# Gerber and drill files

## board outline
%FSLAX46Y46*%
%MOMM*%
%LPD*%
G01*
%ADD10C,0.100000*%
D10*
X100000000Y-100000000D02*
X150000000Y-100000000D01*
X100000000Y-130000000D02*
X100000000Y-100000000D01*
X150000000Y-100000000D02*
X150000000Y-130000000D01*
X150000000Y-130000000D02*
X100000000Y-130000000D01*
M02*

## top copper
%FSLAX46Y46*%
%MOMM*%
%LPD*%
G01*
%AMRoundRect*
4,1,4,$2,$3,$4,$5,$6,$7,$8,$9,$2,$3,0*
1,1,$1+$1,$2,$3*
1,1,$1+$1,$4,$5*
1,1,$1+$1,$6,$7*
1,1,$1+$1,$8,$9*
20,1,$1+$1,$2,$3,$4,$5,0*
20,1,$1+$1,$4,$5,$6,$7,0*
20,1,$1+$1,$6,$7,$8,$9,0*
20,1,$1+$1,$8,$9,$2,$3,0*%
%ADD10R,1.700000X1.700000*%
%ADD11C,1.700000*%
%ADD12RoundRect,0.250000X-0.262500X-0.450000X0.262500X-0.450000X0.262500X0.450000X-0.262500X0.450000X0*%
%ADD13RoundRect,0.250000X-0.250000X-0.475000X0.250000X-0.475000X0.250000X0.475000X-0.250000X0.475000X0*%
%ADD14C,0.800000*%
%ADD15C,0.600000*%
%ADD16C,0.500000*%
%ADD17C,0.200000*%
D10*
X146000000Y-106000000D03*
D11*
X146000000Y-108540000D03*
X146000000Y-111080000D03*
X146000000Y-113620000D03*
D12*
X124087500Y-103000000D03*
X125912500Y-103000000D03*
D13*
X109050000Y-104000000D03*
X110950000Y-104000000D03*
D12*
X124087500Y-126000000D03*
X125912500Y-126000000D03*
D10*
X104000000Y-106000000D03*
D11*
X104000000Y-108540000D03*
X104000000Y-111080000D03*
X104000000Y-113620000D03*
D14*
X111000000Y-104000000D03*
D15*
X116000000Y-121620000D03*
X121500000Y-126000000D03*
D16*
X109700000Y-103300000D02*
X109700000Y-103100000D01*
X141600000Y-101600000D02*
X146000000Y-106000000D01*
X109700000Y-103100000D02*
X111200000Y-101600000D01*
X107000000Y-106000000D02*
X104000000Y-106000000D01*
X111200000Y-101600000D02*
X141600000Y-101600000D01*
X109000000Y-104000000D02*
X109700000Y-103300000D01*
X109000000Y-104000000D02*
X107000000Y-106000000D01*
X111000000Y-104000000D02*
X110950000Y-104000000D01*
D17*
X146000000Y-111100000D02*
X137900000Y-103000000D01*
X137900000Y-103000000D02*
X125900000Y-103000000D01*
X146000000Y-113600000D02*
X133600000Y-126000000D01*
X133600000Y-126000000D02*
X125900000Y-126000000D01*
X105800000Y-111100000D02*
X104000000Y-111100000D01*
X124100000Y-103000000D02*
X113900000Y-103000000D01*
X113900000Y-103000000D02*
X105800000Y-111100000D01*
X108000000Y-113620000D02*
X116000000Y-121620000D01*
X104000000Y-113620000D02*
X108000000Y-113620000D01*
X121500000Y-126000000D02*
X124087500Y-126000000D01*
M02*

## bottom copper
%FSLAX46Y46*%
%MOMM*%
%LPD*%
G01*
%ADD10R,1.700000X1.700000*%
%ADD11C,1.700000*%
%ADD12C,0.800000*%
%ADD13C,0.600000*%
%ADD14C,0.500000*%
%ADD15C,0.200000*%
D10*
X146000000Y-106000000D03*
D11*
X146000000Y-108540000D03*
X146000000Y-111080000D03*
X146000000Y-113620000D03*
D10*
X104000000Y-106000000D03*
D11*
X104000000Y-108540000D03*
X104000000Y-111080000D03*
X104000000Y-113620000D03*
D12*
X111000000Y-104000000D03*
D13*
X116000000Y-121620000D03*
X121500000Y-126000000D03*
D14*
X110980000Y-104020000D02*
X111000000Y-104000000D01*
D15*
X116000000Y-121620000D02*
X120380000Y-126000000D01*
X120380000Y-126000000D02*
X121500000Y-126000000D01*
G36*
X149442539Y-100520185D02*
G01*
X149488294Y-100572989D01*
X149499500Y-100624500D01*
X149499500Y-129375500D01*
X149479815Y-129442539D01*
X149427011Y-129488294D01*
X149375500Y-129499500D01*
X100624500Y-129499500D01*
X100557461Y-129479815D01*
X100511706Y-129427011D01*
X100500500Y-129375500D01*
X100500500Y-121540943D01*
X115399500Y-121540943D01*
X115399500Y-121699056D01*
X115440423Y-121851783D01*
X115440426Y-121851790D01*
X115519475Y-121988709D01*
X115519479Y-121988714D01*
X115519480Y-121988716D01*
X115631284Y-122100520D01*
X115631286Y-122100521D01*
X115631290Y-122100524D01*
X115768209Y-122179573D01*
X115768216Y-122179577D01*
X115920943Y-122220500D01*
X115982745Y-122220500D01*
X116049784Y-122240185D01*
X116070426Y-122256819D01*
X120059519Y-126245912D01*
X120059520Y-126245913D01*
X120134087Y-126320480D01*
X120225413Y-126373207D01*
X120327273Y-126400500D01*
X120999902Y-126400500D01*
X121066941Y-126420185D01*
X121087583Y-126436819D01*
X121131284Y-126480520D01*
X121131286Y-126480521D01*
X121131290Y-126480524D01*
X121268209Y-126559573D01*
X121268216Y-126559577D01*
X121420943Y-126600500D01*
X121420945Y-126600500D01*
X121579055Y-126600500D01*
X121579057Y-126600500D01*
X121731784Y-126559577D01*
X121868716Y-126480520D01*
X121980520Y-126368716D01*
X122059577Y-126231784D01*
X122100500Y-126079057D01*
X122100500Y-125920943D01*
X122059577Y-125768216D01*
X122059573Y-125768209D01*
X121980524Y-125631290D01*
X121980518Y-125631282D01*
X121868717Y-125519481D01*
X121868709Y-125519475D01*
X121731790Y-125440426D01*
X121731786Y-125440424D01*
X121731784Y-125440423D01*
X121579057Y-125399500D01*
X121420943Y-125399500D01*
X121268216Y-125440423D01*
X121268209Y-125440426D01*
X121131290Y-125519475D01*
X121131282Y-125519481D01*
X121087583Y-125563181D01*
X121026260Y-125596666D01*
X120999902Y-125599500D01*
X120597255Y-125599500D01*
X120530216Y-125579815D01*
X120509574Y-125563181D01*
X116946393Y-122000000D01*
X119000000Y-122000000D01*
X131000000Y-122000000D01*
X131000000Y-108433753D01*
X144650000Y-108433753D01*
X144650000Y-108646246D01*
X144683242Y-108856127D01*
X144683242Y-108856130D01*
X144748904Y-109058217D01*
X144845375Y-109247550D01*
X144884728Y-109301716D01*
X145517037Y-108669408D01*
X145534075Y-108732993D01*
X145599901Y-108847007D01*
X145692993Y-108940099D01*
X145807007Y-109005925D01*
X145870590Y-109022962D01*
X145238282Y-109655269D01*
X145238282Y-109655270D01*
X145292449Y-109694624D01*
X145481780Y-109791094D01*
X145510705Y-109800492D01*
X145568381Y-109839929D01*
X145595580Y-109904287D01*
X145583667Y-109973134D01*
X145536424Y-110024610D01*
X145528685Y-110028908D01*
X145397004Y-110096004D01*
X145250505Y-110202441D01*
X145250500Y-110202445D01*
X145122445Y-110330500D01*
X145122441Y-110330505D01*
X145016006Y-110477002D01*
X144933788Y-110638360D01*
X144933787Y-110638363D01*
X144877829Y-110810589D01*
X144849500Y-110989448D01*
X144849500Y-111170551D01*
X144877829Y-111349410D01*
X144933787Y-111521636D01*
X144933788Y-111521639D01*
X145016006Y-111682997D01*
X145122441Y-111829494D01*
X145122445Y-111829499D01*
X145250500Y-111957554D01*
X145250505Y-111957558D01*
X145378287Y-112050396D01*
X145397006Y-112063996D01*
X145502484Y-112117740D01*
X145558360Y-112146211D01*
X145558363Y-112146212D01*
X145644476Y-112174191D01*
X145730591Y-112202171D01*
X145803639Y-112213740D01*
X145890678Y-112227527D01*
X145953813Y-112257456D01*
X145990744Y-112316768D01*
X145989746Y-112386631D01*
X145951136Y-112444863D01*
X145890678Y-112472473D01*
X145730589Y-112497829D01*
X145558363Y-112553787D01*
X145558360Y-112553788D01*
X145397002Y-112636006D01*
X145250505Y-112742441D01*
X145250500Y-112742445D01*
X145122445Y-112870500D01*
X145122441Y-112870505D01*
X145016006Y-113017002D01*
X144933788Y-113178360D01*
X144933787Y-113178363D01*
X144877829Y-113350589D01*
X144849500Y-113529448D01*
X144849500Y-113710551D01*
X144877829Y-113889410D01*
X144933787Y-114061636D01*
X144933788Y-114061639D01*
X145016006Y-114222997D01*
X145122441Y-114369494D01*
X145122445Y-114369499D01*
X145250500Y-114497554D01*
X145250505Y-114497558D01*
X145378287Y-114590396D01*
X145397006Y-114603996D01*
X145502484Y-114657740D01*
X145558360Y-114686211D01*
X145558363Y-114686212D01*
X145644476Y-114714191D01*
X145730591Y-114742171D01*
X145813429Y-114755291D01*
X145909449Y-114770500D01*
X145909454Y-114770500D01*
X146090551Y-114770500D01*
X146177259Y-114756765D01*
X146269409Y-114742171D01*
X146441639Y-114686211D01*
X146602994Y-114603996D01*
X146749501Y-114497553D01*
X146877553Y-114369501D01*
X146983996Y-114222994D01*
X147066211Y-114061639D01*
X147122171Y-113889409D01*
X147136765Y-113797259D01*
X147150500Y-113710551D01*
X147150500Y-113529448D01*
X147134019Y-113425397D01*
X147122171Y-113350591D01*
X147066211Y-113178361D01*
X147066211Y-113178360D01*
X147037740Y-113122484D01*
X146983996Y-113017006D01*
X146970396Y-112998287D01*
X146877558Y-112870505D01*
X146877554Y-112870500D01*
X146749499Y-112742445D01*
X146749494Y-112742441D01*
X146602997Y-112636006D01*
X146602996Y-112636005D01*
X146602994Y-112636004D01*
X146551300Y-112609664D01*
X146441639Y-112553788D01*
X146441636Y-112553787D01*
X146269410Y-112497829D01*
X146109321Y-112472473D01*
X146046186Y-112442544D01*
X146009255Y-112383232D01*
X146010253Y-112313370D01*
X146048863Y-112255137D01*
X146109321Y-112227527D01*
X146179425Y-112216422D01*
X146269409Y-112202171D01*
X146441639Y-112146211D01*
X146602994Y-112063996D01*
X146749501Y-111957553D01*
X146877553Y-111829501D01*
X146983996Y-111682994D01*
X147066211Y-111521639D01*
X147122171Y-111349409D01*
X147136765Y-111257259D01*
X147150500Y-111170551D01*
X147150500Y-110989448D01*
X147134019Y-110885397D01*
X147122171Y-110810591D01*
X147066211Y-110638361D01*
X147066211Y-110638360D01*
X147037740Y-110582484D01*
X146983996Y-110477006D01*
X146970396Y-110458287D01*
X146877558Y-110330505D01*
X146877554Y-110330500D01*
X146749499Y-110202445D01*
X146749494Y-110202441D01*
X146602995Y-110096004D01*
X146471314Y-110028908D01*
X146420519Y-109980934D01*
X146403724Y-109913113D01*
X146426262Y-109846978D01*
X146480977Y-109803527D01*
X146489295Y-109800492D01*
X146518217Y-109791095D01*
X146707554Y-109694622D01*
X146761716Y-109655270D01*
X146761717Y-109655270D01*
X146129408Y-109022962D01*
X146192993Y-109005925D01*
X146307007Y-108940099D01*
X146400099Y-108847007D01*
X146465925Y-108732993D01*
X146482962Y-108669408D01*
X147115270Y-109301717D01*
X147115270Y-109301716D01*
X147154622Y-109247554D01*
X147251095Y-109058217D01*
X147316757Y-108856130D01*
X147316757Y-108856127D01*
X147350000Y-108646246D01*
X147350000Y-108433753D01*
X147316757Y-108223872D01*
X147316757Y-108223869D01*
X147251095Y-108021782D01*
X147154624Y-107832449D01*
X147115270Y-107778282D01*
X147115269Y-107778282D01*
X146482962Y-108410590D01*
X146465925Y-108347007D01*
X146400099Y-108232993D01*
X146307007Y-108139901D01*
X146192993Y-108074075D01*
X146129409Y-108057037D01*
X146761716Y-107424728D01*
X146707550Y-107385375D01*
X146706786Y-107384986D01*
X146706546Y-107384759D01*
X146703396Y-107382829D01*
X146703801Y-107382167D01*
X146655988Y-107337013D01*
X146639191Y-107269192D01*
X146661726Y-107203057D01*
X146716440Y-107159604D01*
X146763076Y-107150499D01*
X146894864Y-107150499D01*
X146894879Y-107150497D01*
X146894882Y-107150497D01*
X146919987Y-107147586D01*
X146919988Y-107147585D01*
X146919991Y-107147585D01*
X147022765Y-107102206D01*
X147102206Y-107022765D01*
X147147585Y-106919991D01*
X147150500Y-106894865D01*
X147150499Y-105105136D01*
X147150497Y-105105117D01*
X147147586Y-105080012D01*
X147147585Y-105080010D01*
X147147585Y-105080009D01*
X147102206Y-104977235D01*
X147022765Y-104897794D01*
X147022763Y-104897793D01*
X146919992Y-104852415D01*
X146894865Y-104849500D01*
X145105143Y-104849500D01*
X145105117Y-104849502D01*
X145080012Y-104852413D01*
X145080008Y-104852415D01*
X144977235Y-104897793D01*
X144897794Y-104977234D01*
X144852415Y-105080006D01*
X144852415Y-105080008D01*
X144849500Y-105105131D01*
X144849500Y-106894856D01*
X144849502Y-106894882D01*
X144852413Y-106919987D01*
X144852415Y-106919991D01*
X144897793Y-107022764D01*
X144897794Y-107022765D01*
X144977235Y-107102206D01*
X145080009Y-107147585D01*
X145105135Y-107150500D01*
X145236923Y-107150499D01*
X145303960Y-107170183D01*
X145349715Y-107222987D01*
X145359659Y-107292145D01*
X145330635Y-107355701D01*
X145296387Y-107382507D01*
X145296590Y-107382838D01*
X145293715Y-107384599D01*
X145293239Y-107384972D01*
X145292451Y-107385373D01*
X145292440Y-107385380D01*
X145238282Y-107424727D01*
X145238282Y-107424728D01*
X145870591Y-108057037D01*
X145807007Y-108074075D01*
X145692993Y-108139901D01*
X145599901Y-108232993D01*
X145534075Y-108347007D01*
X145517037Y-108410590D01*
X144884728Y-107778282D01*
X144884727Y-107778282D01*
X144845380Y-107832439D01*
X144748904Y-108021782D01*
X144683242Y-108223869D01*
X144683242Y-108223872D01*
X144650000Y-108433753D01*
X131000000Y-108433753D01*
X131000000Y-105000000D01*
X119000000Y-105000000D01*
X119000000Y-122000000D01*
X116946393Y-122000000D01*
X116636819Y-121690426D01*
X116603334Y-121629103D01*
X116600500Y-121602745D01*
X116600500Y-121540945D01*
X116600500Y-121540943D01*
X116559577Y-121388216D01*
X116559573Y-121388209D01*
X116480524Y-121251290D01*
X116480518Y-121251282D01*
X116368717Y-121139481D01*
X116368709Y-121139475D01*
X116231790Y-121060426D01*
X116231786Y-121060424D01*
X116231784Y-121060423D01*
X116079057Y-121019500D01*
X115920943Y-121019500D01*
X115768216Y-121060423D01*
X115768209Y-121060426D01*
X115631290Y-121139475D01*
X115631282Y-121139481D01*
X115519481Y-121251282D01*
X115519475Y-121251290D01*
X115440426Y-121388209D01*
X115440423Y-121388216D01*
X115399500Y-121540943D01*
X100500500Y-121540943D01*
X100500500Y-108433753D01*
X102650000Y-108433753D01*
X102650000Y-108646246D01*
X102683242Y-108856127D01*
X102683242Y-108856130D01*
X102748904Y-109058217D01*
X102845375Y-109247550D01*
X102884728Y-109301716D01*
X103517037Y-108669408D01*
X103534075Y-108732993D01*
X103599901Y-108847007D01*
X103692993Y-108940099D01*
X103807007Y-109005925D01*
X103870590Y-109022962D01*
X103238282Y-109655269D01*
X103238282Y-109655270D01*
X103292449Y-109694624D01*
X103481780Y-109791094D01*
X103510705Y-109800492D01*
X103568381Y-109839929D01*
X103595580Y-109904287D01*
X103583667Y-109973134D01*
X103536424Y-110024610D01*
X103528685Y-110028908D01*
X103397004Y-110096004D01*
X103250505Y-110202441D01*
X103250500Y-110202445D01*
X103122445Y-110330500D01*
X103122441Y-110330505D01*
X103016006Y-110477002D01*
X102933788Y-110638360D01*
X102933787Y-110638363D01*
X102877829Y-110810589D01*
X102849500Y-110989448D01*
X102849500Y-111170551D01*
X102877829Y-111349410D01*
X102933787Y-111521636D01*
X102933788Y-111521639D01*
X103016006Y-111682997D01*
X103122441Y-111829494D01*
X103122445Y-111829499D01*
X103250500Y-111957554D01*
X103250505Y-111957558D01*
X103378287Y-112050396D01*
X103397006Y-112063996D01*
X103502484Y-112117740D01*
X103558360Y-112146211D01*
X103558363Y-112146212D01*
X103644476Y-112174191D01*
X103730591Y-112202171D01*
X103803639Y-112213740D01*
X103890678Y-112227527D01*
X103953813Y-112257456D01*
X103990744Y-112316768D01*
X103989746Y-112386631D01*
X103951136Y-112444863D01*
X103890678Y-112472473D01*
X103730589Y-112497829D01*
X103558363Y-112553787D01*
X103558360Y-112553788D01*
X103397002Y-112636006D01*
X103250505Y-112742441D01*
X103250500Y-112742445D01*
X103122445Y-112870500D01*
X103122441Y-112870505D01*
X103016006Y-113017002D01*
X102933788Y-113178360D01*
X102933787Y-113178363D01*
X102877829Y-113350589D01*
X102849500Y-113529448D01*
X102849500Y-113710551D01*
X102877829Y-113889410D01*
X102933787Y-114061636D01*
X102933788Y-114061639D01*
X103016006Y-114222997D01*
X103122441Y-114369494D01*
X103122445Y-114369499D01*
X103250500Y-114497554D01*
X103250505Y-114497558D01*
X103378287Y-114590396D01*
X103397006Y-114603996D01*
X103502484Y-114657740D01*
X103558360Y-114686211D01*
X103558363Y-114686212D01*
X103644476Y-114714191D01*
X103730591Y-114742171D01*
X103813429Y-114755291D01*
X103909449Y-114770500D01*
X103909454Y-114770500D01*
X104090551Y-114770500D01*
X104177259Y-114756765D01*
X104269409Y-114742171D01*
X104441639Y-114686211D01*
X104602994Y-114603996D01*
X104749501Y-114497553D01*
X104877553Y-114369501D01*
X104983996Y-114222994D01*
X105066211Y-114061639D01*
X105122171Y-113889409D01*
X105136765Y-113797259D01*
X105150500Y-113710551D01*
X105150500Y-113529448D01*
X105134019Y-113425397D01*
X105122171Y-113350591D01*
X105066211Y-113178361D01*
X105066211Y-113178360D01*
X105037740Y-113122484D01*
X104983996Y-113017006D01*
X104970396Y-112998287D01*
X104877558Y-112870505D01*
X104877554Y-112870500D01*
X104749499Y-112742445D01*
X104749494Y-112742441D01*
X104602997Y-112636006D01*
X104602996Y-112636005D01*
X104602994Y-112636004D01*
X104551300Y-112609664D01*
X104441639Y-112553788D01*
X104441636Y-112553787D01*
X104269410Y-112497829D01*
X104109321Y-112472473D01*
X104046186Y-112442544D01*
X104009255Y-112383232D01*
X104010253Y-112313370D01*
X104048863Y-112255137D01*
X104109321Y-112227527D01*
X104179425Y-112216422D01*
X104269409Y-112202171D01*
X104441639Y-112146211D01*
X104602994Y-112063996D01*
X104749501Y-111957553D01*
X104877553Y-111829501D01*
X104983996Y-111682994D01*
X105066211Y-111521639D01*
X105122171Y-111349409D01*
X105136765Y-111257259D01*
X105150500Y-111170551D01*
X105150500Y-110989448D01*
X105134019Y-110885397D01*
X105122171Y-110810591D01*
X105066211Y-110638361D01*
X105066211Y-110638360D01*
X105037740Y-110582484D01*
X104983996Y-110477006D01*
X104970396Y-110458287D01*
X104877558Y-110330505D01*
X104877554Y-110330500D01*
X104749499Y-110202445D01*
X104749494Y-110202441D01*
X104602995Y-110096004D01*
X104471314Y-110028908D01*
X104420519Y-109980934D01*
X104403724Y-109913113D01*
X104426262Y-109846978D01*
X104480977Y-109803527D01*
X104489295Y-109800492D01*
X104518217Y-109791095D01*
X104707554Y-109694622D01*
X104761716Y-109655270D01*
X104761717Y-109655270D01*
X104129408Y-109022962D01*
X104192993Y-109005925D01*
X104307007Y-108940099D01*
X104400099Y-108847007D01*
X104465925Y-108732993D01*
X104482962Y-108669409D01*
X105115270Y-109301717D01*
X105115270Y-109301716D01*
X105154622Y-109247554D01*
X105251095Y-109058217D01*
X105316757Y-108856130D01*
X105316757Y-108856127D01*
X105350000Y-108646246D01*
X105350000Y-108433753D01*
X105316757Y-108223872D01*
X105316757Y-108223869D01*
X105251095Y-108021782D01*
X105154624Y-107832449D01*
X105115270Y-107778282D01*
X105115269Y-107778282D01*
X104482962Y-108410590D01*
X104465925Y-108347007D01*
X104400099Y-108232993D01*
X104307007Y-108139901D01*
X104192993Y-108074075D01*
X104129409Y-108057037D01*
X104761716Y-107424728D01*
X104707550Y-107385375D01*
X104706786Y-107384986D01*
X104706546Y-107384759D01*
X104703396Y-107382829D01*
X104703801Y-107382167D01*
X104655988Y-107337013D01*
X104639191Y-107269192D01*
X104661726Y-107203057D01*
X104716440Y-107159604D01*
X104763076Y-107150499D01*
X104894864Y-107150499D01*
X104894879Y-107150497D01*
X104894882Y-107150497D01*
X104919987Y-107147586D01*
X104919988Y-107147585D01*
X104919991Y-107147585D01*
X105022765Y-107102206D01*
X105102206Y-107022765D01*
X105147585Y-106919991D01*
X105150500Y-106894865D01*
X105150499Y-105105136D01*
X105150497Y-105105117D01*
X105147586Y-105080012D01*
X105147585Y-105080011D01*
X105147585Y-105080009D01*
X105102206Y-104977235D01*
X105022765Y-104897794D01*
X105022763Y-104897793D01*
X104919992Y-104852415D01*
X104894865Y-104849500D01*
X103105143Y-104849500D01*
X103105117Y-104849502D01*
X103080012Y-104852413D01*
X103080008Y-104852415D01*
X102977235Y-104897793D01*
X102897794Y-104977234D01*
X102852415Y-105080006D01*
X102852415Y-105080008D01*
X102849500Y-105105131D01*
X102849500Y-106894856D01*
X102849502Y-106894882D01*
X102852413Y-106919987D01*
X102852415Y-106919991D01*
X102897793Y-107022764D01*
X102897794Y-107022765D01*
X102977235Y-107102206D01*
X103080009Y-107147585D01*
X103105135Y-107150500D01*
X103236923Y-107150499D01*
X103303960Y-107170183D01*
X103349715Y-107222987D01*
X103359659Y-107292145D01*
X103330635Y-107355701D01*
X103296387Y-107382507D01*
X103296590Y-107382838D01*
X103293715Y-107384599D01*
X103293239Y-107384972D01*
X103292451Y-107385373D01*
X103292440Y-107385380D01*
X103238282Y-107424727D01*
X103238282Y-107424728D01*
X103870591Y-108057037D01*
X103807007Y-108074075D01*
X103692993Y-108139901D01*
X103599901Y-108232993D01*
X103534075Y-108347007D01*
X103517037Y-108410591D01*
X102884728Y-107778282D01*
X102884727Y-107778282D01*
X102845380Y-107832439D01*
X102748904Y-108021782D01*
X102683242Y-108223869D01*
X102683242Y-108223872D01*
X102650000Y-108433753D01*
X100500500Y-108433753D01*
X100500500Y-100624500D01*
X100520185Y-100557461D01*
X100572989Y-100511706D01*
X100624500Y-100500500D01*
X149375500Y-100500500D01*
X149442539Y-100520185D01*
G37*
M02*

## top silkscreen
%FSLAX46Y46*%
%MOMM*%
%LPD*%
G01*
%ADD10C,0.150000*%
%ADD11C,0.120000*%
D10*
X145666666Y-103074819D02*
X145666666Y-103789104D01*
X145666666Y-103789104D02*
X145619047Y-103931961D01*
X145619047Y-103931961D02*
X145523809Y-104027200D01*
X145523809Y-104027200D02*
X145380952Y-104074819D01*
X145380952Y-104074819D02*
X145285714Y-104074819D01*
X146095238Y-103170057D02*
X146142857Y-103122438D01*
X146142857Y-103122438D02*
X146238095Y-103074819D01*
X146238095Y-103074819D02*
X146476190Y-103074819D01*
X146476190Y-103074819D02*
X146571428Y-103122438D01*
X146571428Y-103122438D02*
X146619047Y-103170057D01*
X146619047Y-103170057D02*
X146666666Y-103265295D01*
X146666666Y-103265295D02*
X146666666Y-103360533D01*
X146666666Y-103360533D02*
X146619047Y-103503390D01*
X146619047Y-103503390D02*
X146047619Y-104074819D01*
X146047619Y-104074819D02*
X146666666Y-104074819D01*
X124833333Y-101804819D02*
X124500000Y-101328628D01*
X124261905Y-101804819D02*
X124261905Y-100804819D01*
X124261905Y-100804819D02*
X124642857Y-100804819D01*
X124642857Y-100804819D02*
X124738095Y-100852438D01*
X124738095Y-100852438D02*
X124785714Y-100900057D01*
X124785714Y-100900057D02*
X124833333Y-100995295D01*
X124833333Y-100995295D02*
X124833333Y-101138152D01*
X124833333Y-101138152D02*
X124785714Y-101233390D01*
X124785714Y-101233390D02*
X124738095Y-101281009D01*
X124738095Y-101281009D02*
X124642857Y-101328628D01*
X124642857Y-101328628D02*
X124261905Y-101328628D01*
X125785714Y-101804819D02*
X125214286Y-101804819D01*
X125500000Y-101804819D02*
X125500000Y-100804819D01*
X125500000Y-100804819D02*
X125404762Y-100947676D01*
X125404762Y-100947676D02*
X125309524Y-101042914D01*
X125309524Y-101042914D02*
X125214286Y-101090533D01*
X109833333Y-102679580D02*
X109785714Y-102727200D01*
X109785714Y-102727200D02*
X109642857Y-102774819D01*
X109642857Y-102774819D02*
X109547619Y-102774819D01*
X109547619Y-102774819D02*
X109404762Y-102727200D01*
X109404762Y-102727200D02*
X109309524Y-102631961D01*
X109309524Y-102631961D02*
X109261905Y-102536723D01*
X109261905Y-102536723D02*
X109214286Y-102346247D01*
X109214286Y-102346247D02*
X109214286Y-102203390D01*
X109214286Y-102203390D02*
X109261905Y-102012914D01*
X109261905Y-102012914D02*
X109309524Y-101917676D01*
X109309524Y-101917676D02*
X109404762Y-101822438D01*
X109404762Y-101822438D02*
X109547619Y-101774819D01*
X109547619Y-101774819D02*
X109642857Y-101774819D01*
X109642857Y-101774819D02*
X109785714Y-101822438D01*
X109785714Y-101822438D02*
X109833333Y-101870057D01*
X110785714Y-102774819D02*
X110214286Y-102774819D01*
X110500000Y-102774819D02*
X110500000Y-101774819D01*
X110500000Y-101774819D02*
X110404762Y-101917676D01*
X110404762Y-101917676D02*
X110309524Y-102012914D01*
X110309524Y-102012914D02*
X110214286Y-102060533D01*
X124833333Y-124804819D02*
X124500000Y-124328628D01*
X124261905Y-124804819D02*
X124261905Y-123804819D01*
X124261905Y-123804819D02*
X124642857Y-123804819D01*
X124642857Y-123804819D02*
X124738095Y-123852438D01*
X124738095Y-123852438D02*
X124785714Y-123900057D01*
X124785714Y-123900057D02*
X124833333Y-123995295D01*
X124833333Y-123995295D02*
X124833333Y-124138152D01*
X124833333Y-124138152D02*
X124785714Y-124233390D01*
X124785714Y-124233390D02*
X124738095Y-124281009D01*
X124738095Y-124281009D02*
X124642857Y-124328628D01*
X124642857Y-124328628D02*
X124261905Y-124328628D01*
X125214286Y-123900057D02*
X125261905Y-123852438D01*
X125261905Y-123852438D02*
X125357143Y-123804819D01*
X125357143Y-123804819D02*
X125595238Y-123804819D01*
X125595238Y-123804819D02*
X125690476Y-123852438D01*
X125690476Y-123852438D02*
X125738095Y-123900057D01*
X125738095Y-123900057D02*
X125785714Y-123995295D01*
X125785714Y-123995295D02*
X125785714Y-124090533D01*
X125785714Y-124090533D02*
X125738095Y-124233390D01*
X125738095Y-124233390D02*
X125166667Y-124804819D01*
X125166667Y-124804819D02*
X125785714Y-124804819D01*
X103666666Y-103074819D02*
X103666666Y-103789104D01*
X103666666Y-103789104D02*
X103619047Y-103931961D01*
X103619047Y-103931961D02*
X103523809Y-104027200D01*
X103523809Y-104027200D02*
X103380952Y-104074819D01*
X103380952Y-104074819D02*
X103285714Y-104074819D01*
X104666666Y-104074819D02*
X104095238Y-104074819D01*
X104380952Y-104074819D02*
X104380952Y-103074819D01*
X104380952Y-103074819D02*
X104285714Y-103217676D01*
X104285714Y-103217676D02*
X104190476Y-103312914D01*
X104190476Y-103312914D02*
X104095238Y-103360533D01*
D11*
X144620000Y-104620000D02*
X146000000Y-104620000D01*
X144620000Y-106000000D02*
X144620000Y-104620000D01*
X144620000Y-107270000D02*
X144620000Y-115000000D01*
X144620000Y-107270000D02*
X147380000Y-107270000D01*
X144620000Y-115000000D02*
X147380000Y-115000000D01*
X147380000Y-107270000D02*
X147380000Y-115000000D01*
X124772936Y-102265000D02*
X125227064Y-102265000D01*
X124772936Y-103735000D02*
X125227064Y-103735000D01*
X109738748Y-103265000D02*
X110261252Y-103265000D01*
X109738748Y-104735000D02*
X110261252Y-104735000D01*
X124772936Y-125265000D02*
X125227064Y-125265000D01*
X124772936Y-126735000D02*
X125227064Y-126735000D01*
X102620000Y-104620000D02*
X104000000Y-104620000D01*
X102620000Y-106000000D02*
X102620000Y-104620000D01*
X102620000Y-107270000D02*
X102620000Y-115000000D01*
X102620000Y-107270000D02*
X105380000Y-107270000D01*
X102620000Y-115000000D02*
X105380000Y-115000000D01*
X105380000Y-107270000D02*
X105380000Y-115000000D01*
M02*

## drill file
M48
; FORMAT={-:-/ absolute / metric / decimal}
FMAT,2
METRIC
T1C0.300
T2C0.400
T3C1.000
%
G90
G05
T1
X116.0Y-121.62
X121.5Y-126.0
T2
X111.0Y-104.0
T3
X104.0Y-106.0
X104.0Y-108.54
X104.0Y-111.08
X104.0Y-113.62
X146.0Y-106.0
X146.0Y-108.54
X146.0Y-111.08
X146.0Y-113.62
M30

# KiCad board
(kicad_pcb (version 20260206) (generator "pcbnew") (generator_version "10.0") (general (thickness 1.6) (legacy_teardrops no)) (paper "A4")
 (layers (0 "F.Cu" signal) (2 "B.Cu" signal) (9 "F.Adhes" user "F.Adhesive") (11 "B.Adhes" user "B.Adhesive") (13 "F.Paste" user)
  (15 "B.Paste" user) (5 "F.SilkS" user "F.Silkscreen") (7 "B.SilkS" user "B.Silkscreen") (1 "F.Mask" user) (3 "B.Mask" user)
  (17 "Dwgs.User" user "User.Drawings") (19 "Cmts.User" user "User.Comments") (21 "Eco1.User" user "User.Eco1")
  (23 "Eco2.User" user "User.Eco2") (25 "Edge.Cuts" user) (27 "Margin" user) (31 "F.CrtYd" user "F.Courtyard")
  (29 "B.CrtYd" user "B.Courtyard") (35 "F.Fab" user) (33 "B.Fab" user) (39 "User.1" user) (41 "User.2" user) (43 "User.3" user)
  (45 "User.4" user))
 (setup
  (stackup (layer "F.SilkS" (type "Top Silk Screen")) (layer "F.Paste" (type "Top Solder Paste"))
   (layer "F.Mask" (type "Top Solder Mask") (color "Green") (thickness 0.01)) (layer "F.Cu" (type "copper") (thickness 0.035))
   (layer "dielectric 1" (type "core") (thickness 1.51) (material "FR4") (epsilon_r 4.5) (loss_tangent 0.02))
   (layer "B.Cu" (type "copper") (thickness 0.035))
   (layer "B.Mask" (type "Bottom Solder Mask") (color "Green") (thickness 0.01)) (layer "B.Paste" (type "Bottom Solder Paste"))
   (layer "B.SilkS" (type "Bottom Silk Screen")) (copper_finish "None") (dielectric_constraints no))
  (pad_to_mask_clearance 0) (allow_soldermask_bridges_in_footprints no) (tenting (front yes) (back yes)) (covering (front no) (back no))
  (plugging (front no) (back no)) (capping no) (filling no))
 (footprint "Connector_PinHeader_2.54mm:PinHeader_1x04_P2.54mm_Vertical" (layer "F.Cu") (at 146 106)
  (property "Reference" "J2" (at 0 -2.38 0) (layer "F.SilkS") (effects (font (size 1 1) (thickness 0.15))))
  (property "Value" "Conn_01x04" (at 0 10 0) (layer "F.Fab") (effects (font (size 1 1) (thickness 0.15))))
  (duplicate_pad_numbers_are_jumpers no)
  (fp_line (start -1.38 -1.38) (end 0 -1.38) (stroke (width 0.12) (type solid)) (layer "F.SilkS"))
  (fp_line (start -1.38 0) (end -1.38 -1.38) (stroke (width 0.12) (type solid)) (layer "F.SilkS"))
  (fp_line (start -1.38 1.27) (end -1.38 9) (stroke (width 0.12) (type solid)) (layer "F.SilkS"))
  (fp_line (start -1.38 1.27) (end 1.38 1.27) (stroke (width 0.12) (type solid)) (layer "F.SilkS"))
  (fp_line (start -1.38 9) (end 1.38 9) (stroke (width 0.12) (type solid)) (layer "F.SilkS"))
  (fp_line (start 1.38 1.27) (end 1.38 9) (stroke (width 0.12) (type solid)) (layer "F.SilkS"))
  (pad "1" thru_hole rect (at 0 0) (size 1.7 1.7) (drill 1) (layers "*.Cu" "*.Mask") (remove_unused_layers no) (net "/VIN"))
  (pad "2" thru_hole circle (at 0 2.54) (size 1.7 1.7) (drill 1) (layers "*.Cu" "*.Mask") (remove_unused_layers no) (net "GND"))
  (pad "3" thru_hole circle (at 0 5.08) (size 1.7 1.7) (drill 1) (layers "*.Cu" "*.Mask") (remove_unused_layers no) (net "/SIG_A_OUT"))
  (pad "4" thru_hole circle (at 0 7.62) (size 1.7 1.7) (drill 1) (layers "*.Cu" "*.Mask") (remove_unused_layers no) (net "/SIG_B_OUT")))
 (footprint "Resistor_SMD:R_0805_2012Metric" (layer "F.Cu") (at 125 103)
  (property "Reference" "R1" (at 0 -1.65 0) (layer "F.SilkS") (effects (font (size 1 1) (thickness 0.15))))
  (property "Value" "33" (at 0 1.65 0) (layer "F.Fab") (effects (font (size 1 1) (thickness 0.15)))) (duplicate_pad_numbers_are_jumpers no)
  (fp_line (start -0.227064 -0.735) (end 0.227064 -0.735) (stroke (width 0.12) (type solid)) (layer "F.SilkS"))
  (fp_line (start -0.227064 0.735) (end 0.227064 0.735) (stroke (width 0.12) (type solid)) (layer "F.SilkS"))
  (pad "1" smd roundrect (at -0.9125 0) (size 1.025 1.4) (layers "F.Cu" "F.Mask" "F.Paste") (roundrect_rratio 0.243902) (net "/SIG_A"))
  (pad "2" smd roundrect (at 0.9125 0) (size 1.025 1.4) (layers "F.Cu" "F.Mask" "F.Paste") (roundrect_rratio 0.243902) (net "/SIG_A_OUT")))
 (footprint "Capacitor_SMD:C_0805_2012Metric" (layer "F.Cu") (at 110 104)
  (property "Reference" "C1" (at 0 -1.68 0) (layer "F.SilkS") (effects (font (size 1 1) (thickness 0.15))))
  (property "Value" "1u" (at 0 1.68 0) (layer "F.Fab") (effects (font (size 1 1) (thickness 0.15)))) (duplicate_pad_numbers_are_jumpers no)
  (fp_line (start -0.261252 -0.735) (end 0.261252 -0.735) (stroke (width 0.12) (type solid)) (layer "F.SilkS"))
  (fp_line (start -0.261252 0.735) (end 0.261252 0.735) (stroke (width 0.12) (type solid)) (layer "F.SilkS"))
  (pad "1" smd roundrect (at -0.95 0) (size 1 1.45) (layers "F.Cu" "F.Mask" "F.Paste") (roundrect_rratio 0.25) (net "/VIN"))
  (pad "2" smd roundrect (at 0.95 0) (size 1 1.45) (layers "F.Cu" "F.Mask" "F.Paste") (roundrect_rratio 0.25) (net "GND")))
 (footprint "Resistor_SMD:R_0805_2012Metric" (layer "F.Cu") (at 125 126)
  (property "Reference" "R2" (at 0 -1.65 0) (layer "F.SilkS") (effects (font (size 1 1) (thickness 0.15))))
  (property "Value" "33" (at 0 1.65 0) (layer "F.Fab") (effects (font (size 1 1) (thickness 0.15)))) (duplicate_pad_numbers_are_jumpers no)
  (fp_line (start -0.227064 -0.735) (end 0.227064 -0.735) (stroke (width 0.12) (type solid)) (layer "F.SilkS"))
  (fp_line (start -0.227064 0.735) (end 0.227064 0.735) (stroke (width 0.12) (type solid)) (layer "F.SilkS"))
  (pad "1" smd roundrect (at -0.9125 0) (size 1.025 1.4) (layers "F.Cu" "F.Mask" "F.Paste") (roundrect_rratio 0.243902) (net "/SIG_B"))
  (pad "2" smd roundrect (at 0.9125 0) (size 1.025 1.4) (layers "F.Cu" "F.Mask" "F.Paste") (roundrect_rratio 0.243902) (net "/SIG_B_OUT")))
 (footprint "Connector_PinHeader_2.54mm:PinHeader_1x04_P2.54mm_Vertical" (layer "F.Cu") (at 104 106)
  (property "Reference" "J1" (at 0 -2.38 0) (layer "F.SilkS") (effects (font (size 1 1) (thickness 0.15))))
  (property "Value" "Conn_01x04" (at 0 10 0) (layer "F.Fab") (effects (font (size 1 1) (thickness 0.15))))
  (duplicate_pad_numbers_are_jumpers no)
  (fp_line (start -1.38 -1.38) (end 0 -1.38) (stroke (width 0.12) (type solid)) (layer "F.SilkS"))
  (fp_line (start -1.38 0) (end -1.38 -1.38) (stroke (width 0.12) (type solid)) (layer "F.SilkS"))
  (fp_line (start -1.38 1.27) (end -1.38 9) (stroke (width 0.12) (type solid)) (layer "F.SilkS"))
  (fp_line (start -1.38 1.27) (end 1.38 1.27) (stroke (width 0.12) (type solid)) (layer "F.SilkS"))
  (fp_line (start -1.38 9) (end 1.38 9) (stroke (width 0.12) (type solid)) (layer "F.SilkS"))
  (fp_line (start 1.38 1.27) (end 1.38 9) (stroke (width 0.12) (type solid)) (layer "F.SilkS"))
  (pad "1" thru_hole rect (at 0 0) (size 1.7 1.7) (drill 1) (layers "*.Cu" "*.Mask") (remove_unused_layers no) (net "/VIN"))
  (pad "2" thru_hole circle (at 0 2.54) (size 1.7 1.7) (drill 1) (layers "*.Cu" "*.Mask") (remove_unused_layers no) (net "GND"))
  (pad "3" thru_hole circle (at 0 5.08) (size 1.7 1.7) (drill 1) (layers "*.Cu" "*.Mask") (remove_unused_layers no) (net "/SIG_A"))
  (pad "4" thru_hole circle (at 0 7.62) (size 1.7 1.7) (drill 1) (layers "*.Cu" "*.Mask") (remove_unused_layers no) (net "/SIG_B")))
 (gr_line (start 100 100) (end 150 100) (stroke (width 0.1) (type default)) (layer "Edge.Cuts"))
 (gr_line (start 100 130) (end 100 100) (stroke (width 0.1) (type default)) (layer "Edge.Cuts"))
 (gr_line (start 150 100) (end 150 130) (stroke (width 0.1) (type default)) (layer "Edge.Cuts"))
 (gr_line (start 150 130) (end 100 130) (stroke (width 0.1) (type default)) (layer "Edge.Cuts"))
 (segment (start 109.7 103.3) (end 109.7 103.1) (width 0.5) (layer "F.Cu") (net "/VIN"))
 (segment (start 141.6 101.6) (end 146 106) (width 0.5) (layer "F.Cu") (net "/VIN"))
 (segment (start 109.7 103.1) (end 111.2 101.6) (width 0.5) (layer "F.Cu") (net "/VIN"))
 (segment (start 107 106) (end 104 106) (width 0.5) (layer "F.Cu") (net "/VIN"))
 (segment (start 111.2 101.6) (end 141.6 101.6) (width 0.5) (layer "F.Cu") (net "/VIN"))
 (segment (start 109 104) (end 109.7 103.3) (width 0.5) (layer "F.Cu") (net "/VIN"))
 (segment (start 109 104) (end 107 106) (width 0.5) (layer "F.Cu") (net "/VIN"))
 (segment (start 111 104) (end 110.95 104) (width 0.5) (layer "F.Cu") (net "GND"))
 (via (at 111 104) (size 0.8) (drill 0.4) (layers "F.Cu" "B.Cu") (capping yes) (filling yes) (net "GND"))
 (segment (start 110.98 104.02) (end 111 104) (width 0.5) (layer "B.Cu") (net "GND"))
 (segment (start 146 111.1) (end 137.9 103) (width 0.2) (layer "F.Cu") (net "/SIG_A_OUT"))
 (segment (start 137.9 103) (end 125.9 103) (width 0.2) (layer "F.Cu") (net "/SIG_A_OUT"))
 (segment (start 146 113.6) (end 133.6 126) (width 0.2) (layer "F.Cu") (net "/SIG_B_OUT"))
 (segment (start 133.6 126) (end 125.9 126) (width 0.2) (layer "F.Cu") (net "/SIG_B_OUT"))
 (segment (start 105.8 111.1) (end 104 111.1) (width 0.2) (layer "F.Cu") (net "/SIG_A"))
 (segment (start 124.1 103) (end 113.9 103) (width 0.2) (layer "F.Cu") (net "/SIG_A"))
 (segment (start 113.9 103) (end 105.8 111.1) (width 0.2) (layer "F.Cu") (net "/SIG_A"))
 (segment (start 108 113.62) (end 116 121.62) (width 0.2) (locked yes) (layer "F.Cu") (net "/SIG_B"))
 (segment (start 104 113.62) (end 108 113.62) (width 0.2) (locked yes) (layer "F.Cu") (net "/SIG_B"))
 (segment (start 121.5 126) (end 124.0875 126) (width 0.2) (locked yes) (layer "F.Cu") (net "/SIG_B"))
 (via (at 116 121.62) (size 0.6) (drill 0.3) (layers "F.Cu" "B.Cu") (locked yes) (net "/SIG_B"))
 (via (at 121.5 126) (size 0.6) (drill 0.3) (layers "F.Cu" "B.Cu") (locked yes) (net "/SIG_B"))
 (segment (start 116 121.62) (end 120.38 126) (width 0.2) (locked yes) (layer "B.Cu") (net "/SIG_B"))
 (segment (start 120.38 126) (end 121.5 126) (width 0.2) (locked yes) (layer "B.Cu") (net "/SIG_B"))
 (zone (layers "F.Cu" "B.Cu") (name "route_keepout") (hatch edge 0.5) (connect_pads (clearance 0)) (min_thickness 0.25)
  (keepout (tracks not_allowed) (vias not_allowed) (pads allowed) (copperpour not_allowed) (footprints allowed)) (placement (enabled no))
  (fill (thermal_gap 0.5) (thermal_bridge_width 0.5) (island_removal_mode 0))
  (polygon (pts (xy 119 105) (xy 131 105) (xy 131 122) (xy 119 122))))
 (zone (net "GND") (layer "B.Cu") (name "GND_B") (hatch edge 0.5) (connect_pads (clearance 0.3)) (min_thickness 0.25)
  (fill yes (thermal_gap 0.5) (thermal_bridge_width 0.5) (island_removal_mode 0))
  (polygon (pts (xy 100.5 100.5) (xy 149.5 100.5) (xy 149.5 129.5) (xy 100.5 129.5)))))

